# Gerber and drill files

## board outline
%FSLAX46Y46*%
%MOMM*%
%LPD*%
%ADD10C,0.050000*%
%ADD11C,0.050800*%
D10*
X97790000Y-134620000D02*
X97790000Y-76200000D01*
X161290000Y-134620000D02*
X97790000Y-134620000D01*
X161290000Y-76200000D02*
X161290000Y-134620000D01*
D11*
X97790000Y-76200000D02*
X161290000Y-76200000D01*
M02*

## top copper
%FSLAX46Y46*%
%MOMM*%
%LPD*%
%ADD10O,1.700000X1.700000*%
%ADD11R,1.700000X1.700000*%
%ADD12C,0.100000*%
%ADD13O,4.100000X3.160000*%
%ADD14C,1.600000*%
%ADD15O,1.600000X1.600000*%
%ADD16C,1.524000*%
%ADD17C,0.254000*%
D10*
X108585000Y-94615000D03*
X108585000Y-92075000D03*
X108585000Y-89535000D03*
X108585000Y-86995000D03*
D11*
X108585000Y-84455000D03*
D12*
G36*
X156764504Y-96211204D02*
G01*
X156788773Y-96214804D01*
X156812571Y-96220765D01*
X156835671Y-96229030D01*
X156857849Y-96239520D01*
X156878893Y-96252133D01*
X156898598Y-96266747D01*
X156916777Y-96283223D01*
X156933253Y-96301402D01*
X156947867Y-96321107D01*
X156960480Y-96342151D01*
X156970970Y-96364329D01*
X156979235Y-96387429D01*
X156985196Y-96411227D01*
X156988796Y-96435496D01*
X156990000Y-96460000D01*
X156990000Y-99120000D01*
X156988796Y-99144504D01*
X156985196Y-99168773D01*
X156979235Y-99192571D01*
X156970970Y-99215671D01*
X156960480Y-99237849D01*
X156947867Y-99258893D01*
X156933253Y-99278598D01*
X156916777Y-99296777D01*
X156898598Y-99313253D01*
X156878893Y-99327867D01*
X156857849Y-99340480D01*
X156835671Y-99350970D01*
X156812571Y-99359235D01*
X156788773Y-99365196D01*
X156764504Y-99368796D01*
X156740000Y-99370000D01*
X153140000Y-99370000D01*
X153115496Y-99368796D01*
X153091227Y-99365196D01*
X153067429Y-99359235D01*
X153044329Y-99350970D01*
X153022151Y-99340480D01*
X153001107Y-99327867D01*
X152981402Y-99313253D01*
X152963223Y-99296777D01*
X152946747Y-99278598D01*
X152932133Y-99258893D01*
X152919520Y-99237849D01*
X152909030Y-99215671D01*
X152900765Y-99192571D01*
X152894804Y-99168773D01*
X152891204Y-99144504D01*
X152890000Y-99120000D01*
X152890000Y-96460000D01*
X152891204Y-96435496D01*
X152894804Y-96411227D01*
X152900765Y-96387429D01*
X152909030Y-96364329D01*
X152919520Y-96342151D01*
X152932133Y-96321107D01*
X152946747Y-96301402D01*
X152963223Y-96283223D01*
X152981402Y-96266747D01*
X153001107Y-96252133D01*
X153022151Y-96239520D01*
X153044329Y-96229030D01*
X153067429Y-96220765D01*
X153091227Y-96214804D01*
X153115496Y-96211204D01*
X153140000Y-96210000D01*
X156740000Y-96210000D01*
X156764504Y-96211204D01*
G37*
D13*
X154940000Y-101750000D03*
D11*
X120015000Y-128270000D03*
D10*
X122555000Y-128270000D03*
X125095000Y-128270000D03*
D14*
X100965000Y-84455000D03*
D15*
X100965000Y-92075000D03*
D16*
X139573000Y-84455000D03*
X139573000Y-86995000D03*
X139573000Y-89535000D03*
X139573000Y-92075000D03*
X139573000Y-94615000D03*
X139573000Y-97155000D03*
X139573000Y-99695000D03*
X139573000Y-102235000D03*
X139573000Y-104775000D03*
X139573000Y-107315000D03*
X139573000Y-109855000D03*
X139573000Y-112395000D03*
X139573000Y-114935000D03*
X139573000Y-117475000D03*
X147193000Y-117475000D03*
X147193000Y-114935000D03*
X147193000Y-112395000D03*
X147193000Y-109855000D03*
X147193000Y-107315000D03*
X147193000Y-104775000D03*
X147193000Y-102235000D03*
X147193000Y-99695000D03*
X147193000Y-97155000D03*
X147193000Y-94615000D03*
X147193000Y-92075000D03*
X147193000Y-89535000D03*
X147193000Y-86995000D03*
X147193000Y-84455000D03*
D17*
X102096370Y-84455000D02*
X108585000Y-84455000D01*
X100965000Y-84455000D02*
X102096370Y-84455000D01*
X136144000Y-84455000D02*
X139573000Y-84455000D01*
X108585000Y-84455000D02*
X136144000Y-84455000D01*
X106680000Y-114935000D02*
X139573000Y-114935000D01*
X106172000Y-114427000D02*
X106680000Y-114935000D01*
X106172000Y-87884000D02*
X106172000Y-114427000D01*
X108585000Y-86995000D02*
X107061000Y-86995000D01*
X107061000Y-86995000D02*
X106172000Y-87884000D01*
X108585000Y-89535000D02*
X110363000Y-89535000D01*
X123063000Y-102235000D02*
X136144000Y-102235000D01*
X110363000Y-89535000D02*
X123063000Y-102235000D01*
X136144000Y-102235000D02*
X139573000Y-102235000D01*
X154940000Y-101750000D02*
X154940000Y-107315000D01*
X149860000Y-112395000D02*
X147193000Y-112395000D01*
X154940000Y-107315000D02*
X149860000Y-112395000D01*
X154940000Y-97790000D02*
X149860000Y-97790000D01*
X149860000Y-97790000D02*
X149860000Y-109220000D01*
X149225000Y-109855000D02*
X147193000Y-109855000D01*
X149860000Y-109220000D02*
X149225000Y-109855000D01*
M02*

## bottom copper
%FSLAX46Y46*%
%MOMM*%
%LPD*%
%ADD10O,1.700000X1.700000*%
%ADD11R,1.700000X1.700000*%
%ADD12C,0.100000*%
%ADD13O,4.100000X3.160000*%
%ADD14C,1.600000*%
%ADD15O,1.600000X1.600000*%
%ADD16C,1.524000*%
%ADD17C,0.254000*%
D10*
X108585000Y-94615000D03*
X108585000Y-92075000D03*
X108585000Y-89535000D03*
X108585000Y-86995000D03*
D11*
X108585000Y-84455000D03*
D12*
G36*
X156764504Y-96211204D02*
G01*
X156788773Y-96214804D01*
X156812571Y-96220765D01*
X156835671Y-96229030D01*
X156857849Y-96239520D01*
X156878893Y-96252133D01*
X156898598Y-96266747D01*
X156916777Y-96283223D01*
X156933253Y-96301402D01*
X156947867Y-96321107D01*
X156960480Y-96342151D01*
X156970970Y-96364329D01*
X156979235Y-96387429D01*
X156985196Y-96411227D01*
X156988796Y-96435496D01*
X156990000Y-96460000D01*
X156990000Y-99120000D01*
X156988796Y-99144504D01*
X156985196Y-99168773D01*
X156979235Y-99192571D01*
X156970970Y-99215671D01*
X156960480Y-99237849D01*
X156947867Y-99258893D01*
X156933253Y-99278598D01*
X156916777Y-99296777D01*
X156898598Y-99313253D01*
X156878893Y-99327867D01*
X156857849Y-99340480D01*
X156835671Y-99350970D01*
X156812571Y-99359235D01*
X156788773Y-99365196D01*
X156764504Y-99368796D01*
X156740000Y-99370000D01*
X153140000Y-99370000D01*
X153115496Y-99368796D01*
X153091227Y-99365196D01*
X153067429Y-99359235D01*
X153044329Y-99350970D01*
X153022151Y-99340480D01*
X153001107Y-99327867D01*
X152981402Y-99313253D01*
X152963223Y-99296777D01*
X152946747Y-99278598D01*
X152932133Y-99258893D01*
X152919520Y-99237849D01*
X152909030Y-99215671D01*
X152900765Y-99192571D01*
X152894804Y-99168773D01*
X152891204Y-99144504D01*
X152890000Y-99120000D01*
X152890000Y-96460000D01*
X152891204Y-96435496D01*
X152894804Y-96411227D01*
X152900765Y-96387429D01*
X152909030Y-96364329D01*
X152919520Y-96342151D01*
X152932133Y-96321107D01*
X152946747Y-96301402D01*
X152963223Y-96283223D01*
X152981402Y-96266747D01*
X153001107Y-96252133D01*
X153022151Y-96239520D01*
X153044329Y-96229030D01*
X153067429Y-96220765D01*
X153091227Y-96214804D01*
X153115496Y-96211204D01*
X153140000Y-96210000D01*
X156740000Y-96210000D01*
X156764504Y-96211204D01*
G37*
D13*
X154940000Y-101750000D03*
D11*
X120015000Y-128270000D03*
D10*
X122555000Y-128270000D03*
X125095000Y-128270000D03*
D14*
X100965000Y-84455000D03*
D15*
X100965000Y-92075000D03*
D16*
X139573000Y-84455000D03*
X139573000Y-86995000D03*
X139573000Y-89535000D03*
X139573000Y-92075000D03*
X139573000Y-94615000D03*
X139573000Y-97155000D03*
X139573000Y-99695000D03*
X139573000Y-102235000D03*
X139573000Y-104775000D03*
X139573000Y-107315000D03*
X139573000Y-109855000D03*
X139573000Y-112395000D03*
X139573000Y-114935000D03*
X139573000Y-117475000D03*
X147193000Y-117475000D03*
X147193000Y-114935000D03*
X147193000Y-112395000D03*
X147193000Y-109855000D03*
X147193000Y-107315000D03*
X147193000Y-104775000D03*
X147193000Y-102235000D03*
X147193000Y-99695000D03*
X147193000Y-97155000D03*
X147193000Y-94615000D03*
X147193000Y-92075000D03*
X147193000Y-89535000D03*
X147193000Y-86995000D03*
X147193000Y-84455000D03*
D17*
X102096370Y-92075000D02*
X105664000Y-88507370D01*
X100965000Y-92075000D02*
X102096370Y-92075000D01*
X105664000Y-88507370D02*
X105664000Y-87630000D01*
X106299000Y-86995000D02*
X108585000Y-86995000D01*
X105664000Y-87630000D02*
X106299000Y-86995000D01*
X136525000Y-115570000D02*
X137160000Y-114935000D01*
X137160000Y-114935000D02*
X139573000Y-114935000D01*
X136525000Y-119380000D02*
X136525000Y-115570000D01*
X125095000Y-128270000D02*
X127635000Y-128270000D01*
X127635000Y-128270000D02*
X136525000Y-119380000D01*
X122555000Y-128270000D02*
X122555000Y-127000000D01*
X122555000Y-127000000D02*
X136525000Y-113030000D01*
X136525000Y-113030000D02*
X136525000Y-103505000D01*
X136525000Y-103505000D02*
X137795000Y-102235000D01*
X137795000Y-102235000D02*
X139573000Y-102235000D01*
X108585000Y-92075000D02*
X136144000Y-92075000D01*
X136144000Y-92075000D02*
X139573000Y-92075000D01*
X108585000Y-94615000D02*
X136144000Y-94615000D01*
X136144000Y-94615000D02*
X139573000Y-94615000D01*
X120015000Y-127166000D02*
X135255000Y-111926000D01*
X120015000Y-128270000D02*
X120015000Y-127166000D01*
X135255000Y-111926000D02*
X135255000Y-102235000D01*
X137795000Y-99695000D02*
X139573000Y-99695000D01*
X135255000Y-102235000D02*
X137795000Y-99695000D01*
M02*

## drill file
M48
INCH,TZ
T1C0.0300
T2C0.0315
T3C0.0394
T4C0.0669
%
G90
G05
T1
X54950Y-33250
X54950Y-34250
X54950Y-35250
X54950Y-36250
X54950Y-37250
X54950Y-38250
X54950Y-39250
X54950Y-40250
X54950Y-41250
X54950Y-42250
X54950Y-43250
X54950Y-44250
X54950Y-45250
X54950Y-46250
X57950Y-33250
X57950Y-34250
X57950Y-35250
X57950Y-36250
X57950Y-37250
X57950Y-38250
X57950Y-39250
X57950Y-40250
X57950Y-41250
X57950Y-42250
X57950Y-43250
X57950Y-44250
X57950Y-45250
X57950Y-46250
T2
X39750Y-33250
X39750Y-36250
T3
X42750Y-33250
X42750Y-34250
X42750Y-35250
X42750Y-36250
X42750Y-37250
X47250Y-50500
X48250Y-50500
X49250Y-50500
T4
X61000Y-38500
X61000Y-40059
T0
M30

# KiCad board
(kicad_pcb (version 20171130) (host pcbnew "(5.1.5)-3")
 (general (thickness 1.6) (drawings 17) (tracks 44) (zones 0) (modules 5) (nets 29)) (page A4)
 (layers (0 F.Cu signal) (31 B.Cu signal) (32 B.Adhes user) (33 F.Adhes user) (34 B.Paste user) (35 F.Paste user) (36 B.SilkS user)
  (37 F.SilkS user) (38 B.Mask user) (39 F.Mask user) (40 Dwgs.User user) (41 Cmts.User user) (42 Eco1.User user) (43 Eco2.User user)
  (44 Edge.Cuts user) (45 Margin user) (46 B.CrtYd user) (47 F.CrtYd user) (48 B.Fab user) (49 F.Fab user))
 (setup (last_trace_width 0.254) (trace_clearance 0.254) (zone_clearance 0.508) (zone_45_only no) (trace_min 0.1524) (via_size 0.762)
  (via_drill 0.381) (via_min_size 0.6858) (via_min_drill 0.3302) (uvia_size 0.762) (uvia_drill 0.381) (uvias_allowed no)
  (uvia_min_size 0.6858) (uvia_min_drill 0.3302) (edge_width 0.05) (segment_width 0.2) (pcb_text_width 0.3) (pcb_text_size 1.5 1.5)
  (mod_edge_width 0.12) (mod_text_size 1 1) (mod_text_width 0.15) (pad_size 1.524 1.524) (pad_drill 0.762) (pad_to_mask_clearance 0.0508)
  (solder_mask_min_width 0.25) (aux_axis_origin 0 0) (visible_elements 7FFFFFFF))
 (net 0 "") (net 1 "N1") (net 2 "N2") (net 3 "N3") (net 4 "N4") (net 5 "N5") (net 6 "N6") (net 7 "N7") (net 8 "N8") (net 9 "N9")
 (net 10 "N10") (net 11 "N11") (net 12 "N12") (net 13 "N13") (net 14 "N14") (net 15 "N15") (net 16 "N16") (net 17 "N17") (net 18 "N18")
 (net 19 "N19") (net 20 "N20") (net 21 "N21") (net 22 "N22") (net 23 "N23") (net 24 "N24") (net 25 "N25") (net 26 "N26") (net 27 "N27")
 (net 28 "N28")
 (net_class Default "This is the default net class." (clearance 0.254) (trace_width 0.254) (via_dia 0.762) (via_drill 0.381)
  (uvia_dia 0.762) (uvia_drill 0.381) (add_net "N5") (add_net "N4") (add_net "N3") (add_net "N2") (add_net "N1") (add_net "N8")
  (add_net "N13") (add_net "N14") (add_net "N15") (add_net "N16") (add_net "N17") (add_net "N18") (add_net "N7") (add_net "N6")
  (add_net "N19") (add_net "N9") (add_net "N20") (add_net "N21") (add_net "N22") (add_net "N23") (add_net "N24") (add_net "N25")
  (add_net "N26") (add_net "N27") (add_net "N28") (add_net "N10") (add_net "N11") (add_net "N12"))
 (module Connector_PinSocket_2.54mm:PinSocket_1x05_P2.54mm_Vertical (layer F.Cu) (at 108.585 84.455)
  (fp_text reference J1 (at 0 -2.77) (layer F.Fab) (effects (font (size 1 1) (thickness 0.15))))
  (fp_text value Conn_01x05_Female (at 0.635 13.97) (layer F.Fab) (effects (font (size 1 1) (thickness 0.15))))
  (pad 5 thru_hole oval (at 0 10.16) (size 1.7 1.7) (drill 1) (layers *.Cu *.Mask) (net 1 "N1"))
  (pad 4 thru_hole oval (at 0 7.62) (size 1.7 1.7) (drill 1) (layers *.Cu *.Mask) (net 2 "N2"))
  (pad 3 thru_hole oval (at 0 5.08) (size 1.7 1.7) (drill 1) (layers *.Cu *.Mask) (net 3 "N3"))
  (pad 2 thru_hole oval (at 0 2.54) (size 1.7 1.7) (drill 1) (layers *.Cu *.Mask) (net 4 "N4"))
  (pad 1 thru_hole rect (at 0 0) (size 1.7 1.7) (drill 1) (layers *.Cu *.Mask) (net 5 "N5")))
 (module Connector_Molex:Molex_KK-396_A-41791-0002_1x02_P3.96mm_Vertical (layer F.Cu) (at 154.94 97.79 270)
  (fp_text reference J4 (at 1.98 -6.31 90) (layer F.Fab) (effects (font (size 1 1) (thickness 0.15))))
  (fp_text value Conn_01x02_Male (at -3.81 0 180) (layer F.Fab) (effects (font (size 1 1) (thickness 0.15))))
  (pad 1 thru_hole roundrect (at 0 0 270) (size 3.16 4.1) (drill 1.7) (layers *.Cu *.Mask) (roundrect_rratio 0.079114) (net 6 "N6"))
  (pad 2 thru_hole oval (at 3.96 0 270) (size 3.16 4.1) (drill 1.7) (layers *.Cu *.Mask) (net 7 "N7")))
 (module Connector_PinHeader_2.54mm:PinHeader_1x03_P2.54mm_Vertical (layer F.Cu) (at 120.015 128.27 90)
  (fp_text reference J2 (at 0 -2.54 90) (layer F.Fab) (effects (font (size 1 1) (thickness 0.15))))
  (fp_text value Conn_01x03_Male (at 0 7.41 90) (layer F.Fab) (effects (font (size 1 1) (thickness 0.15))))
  (pad 1 thru_hole rect (at 0 0 90) (size 1.7 1.7) (drill 1) (layers *.Cu *.Mask) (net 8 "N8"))
  (pad 2 thru_hole oval (at 0 2.54 90) (size 1.7 1.7) (drill 1) (layers *.Cu *.Mask) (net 3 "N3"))
  (pad 3 thru_hole oval (at 0 5.08 90) (size 1.7 1.7) (drill 1) (layers *.Cu *.Mask) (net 4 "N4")))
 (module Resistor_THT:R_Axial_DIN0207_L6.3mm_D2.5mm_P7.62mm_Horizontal (layer F.Cu) (at 100.965 84.455 270)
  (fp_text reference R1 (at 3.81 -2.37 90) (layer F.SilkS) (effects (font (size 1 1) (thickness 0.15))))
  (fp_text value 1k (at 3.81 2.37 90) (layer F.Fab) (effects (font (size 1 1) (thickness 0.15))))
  (pad 1 thru_hole circle (at 0 0 270) (size 1.6 1.6) (drill 0.8) (layers *.Cu *.Mask) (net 5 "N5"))
  (pad 2 thru_hole oval (at 7.62 0 270) (size 1.6 1.6) (drill 0.8) (layers *.Cu *.Mask) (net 4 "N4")))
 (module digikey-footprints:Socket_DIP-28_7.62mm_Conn (layer F.Cu) (at 139.573 84.455)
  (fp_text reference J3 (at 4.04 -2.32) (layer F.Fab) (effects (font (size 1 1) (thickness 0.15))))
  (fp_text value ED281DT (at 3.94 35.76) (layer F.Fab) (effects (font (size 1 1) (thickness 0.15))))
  (pad 1 thru_hole circle (at 0 0) (size 1.524 1.524) (drill 0.762) (layers *.Cu *.Mask) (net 5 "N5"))
  (pad 2 thru_hole circle (at 0 2.54) (size 1.524 1.524) (drill 0.762) (layers *.Cu *.Mask) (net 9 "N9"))
  (pad 3 thru_hole circle (at 0 5.08) (size 1.524 1.524) (drill 0.762) (layers *.Cu *.Mask) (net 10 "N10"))
  (pad 4 thru_hole circle (at 0 7.62) (size 1.524 1.524) (drill 0.762) (layers *.Cu *.Mask) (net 2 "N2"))
  (pad 5 thru_hole circle (at 0 10.16) (size 1.524 1.524) (drill 0.762) (layers *.Cu *.Mask) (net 1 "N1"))
  (pad 6 thru_hole circle (at 0 12.7) (size 1.524 1.524) (drill 0.762) (layers *.Cu *.Mask) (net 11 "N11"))
  (pad 7 thru_hole circle (at 0 15.24) (size 1.524 1.524) (drill 0.762) (layers *.Cu *.Mask) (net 8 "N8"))
  (pad 8 thru_hole circle (at 0 17.78) (size 1.524 1.524) (drill 0.762) (layers *.Cu *.Mask) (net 3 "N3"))
  (pad 9 thru_hole circle (at 0 20.32) (size 1.524 1.524) (drill 0.762) (layers *.Cu *.Mask) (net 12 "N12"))
  (pad 10 thru_hole circle (at 0 22.86) (size 1.524 1.524) (drill 0.762) (layers *.Cu *.Mask) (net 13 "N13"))
  (pad 11 thru_hole circle (at 0 25.4) (size 1.524 1.524) (drill 0.762) (layers *.Cu *.Mask) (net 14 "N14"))
  (pad 12 thru_hole circle (at 0 27.94) (size 1.524 1.524) (drill 0.762) (layers *.Cu *.Mask) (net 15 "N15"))
  (pad 13 thru_hole circle (at 0 30.48) (size 1.524 1.524) (drill 0.762) (layers *.Cu *.Mask) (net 4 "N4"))
  (pad 14 thru_hole circle (at 0 33.02) (size 1.524 1.524) (drill 0.762) (layers *.Cu *.Mask) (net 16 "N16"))
  (pad 15 thru_hole circle (at 7.62 33.02) (size 1.524 1.524) (drill 0.762) (layers *.Cu *.Mask) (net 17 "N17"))
  (pad 16 thru_hole circle (at 7.62 30.48) (size 1.524 1.524) (drill 0.762) (layers *.Cu *.Mask) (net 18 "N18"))
  (pad 17 thru_hole circle (at 7.62 27.94) (size 1.524 1.524) (drill 0.762) (layers *.Cu *.Mask) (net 7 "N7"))
  (pad 18 thru_hole circle (at 7.62 25.4) (size 1.524 1.524) (drill 0.762) (layers *.Cu *.Mask) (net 6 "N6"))
  (pad 19 thru_hole circle (at 7.62 22.86) (size 1.524 1.524) (drill 0.762) (layers *.Cu *.Mask) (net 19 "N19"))
  (pad 20 thru_hole circle (at 7.62 20.32) (size 1.524 1.524) (drill 0.762) (layers *.Cu *.Mask) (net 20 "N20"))
  (pad 21 thru_hole circle (at 7.62 17.78) (size 1.524 1.524) (drill 0.762) (layers *.Cu *.Mask) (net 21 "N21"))
  (pad 22 thru_hole circle (at 7.62 15.24) (size 1.524 1.524) (drill 0.762) (layers *.Cu *.Mask) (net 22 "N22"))
  (pad 23 thru_hole circle (at 7.62 12.7) (size 1.524 1.524) (drill 0.762) (layers *.Cu *.Mask) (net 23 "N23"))
  (pad 24 thru_hole circle (at 7.62 10.16) (size 1.524 1.524) (drill 0.762) (layers *.Cu *.Mask) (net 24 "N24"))
  (pad 25 thru_hole circle (at 7.62 7.62) (size 1.524 1.524) (drill 0.762) (layers *.Cu *.Mask) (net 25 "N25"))
  (pad 26 thru_hole circle (at 7.62 5.08) (size 1.524 1.524) (drill 0.762) (layers *.Cu *.Mask) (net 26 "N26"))
  (pad 27 thru_hole circle (at 7.62 2.54) (size 1.524 1.524) (drill 0.762) (layers *.Cu *.Mask) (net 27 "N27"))
  (pad 28 thru_hole circle (at 7.62 0) (size 1.524 1.524) (drill 0.762) (layers *.Cu *.Mask) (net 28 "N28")))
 (gr_line (start 97.79 134.62) (end 97.79 76.2) (layer Edge.Cuts) (width 0.05))
 (gr_line (start 161.29 134.62) (end 97.79 134.62) (layer Edge.Cuts) (width 0.05))
 (gr_line (start 161.29 76.2) (end 161.29 134.62) (layer Edge.Cuts) (width 0.05))
 (gr_line (start 97.79 76.2) (end 161.29 76.2) (layer Edge.Cuts) (width 0.0508))
 (segment (start 102.09637 84.455) (end 108.585 84.455) (width 0.254) (layer F.Cu) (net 5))
 (segment (start 100.965 84.455) (end 102.09637 84.455) (width 0.254) (layer F.Cu) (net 5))
 (segment (start 136.144 84.455) (end 139.573 84.455) (width 0.254) (layer F.Cu) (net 5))
 (segment (start 108.585 84.455) (end 136.144 84.455) (width 0.254) (layer F.Cu) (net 5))
 (segment (start 102.09637 92.075) (end 105.664 88.50737) (width 0.254) (layer B.Cu) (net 4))
 (segment (start 100.965 92.075) (end 102.09637 92.075) (width 0.254) (layer B.Cu) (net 4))
 (segment (start 105.664 88.50737) (end 105.664 87.63) (width 0.254) (layer B.Cu) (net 4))
 (segment (start 106.299 86.995) (end 108.585 86.995) (width 0.254) (layer B.Cu) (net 4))
 (segment (start 105.664 87.63) (end 106.299 86.995) (width 0.254) (layer B.Cu) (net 4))
 (segment (start 106.68 114.935) (end 139.573 114.935) (width 0.254) (layer F.Cu) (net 4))
 (segment (start 106.172 114.427) (end 106.68 114.935) (width 0.254) (layer F.Cu) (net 4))
 (segment (start 106.172 87.884) (end 106.172 114.427) (width 0.254) (layer F.Cu) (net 4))
 (segment (start 108.585 86.995) (end 107.061 86.995) (width 0.254) (layer F.Cu) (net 4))
 (segment (start 107.061 86.995) (end 106.172 87.884) (width 0.254) (layer F.Cu) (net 4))
 (segment (start 136.525 115.57) (end 137.16 114.935) (width 0.254) (layer B.Cu) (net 4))
 (segment (start 137.16 114.935) (end 139.573 114.935) (width 0.254) (layer B.Cu) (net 4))
 (segment (start 136.525 119.38) (end 136.525 115.57) (width 0.254) (layer B.Cu) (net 4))
 (segment (start 125.095 128.27) (end 127.635 128.27) (width 0.254) (layer B.Cu) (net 4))
 (segment (start 127.635 128.27) (end 136.525 119.38) (width 0.254) (layer B.Cu) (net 4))
 (segment (start 108.585 89.535) (end 110.363 89.535) (width 0.254) (layer F.Cu) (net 3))
 (segment (start 123.063 102.235) (end 136.144 102.235) (width 0.254) (layer F.Cu) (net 3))
 (segment (start 110.363 89.535) (end 123.063 102.235) (width 0.254) (layer F.Cu) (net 3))
 (segment (start 136.144 102.235) (end 139.573 102.235) (width 0.254) (layer F.Cu) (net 3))
 (segment (start 122.555 128.27) (end 122.555 127) (width 0.254) (layer B.Cu) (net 3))
 (segment (start 122.555 127) (end 136.525 113.03) (width 0.254) (layer B.Cu) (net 3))
 (segment (start 136.525 113.03) (end 136.525 103.505) (width 0.254) (layer B.Cu) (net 3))
 (segment (start 136.525 103.505) (end 137.795 102.235) (width 0.254) (layer B.Cu) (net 3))
 (segment (start 137.795 102.235) (end 139.573 102.235) (width 0.254) (layer B.Cu) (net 3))
 (segment (start 108.585 92.075) (end 136.144 92.075) (width 0.254) (layer B.Cu) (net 2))
 (segment (start 136.144 92.075) (end 139.573 92.075) (width 0.254) (layer B.Cu) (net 2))
 (segment (start 108.585 94.615) (end 136.144 94.615) (width 0.254) (layer B.Cu) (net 1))
 (segment (start 136.144 94.615) (end 139.573 94.615) (width 0.254) (layer B.Cu) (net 1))
 (segment (start 120.015 127.166) (end 135.255 111.926) (width 0.254) (layer B.Cu) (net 8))
 (segment (start 120.015 128.27) (end 120.015 127.166) (width 0.254) (layer B.Cu) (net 8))
 (segment (start 135.255 111.926) (end 135.255 102.235) (width 0.254) (layer B.Cu) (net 8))
 (segment (start 137.795 99.695) (end 139.573 99.695) (width 0.254) (layer B.Cu) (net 8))
 (segment (start 135.255 102.235) (end 137.795 99.695) (width 0.254) (layer B.Cu) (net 8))
 (segment (start 154.94 101.75) (end 154.94 107.315) (width 0.254) (layer F.Cu) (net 7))
 (segment (start 149.86 112.395) (end 147.193 112.395) (width 0.254) (layer F.Cu) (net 7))
 (segment (start 154.94 107.315) (end 149.86 112.395) (width 0.254) (layer F.Cu) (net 7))
 (segment (start 154.94 97.79) (end 149.86 97.79) (width 0.254) (layer F.Cu) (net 6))
 (segment (start 149.86 97.79) (end 149.86 109.22) (width 0.254) (layer F.Cu) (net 6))
 (segment (start 149.225 109.855) (end 147.193 109.855) (width 0.254) (layer F.Cu) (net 6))
 (segment (start 149.86 109.22) (end 149.225 109.855) (width 0.254) (layer F.Cu) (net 6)))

